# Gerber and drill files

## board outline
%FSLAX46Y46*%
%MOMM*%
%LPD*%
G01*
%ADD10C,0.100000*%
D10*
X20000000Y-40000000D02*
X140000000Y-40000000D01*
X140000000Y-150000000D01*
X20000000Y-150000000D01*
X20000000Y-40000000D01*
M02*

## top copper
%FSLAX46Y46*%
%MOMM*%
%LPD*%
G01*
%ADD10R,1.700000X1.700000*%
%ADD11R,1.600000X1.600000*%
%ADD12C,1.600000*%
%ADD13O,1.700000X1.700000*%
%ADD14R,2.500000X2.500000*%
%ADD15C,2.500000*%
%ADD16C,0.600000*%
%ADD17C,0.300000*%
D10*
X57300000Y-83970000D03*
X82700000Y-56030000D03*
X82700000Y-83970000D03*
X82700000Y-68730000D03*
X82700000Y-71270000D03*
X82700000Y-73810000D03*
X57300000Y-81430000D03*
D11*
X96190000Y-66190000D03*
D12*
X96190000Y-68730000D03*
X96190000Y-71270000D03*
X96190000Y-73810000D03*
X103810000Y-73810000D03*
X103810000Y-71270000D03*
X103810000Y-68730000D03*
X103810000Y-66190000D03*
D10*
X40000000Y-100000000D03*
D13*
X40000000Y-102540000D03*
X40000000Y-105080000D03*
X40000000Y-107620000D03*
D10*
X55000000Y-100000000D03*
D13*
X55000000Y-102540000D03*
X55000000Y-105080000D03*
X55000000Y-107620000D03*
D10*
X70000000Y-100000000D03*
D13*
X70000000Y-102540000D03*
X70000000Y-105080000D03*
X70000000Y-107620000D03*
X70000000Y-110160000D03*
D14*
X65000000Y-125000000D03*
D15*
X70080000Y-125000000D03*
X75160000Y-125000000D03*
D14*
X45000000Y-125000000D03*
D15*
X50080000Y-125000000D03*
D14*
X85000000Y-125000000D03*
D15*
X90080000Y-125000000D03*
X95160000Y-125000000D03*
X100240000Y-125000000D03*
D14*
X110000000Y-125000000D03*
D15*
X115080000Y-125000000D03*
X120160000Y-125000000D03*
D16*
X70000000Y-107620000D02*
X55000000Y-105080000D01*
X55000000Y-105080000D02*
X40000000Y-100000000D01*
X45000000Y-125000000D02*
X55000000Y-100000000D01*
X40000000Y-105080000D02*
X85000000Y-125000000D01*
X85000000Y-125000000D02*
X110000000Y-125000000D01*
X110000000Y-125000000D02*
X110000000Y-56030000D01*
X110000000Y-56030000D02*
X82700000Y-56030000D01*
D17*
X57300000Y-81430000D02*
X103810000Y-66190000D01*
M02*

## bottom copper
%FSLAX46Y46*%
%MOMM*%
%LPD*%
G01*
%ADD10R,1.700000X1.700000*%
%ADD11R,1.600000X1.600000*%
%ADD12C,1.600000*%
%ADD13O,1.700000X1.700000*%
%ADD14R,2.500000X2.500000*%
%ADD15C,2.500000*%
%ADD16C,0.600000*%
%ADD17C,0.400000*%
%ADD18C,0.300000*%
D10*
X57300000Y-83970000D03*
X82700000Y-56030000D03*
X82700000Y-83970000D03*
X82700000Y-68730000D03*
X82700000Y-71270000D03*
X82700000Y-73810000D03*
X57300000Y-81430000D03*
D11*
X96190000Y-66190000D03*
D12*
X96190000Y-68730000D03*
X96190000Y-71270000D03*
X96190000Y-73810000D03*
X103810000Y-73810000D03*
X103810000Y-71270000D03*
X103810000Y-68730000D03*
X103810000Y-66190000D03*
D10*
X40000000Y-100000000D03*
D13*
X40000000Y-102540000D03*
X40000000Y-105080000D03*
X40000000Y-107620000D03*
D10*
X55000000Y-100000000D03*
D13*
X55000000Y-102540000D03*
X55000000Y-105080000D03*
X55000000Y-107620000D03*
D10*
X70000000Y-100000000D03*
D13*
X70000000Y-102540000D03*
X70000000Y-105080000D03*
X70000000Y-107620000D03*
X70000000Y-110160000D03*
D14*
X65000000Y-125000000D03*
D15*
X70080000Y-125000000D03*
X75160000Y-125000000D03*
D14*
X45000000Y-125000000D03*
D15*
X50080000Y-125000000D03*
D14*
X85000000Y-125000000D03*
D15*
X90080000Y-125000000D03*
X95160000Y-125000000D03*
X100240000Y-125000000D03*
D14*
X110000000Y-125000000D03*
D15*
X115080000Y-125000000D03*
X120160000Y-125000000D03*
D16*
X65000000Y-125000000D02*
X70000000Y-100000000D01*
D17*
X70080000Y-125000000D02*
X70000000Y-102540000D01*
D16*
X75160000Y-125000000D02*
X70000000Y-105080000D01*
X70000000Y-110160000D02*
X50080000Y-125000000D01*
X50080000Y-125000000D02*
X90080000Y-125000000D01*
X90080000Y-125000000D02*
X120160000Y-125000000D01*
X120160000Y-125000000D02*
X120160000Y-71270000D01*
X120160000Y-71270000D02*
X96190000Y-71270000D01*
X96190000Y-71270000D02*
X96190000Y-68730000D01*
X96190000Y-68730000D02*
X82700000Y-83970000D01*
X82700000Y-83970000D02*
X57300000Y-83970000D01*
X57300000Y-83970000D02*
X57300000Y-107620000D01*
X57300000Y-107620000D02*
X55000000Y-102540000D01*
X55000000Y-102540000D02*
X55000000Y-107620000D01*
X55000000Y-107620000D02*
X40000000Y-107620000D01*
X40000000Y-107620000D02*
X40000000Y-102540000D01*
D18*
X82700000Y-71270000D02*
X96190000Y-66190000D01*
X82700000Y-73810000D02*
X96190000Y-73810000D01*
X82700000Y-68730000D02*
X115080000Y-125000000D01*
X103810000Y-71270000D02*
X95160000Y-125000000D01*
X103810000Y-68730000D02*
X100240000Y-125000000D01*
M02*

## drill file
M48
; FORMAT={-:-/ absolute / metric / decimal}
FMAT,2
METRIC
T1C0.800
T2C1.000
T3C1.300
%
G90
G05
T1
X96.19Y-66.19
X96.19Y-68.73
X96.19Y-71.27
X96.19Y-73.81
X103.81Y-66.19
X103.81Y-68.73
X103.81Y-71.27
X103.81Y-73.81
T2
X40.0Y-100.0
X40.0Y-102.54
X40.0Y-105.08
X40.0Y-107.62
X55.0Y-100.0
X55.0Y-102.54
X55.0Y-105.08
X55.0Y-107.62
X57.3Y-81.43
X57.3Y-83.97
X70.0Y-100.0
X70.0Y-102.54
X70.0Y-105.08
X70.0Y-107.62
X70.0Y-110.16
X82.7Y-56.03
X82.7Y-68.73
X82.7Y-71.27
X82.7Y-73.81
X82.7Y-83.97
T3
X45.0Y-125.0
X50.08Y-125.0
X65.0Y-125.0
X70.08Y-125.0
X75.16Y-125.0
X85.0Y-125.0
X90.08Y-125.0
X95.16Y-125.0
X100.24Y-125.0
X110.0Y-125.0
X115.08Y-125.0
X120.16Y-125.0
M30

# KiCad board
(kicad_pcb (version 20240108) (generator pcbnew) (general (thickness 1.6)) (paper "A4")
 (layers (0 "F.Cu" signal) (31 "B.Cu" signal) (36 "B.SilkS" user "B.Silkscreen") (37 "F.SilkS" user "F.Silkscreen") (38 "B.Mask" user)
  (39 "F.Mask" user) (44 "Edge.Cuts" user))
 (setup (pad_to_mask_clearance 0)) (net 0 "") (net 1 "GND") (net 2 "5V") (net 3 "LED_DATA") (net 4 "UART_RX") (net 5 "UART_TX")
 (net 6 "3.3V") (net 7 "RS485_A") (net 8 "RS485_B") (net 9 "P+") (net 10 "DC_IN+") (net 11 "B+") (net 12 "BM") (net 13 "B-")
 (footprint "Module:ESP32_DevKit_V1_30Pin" (layer "F.Cu") (at 70 70)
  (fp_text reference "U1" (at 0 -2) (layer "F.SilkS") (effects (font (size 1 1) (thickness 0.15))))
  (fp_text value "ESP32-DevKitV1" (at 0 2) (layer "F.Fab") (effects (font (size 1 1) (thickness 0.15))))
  (pad "1" thru_hole rect (at -12.7 13.97) (size 1.7 1.7) (drill 1.0) (layers "*.Cu" "*.Mask") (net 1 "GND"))
  (pad "29" thru_hole rect (at 12.7 -13.97) (size 1.7 1.7) (drill 1.0) (layers "*.Cu" "*.Mask") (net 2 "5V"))
  (pad "30" thru_hole rect (at 12.7 13.97) (size 1.7 1.7) (drill 1.0) (layers "*.Cu" "*.Mask") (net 1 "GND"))
  (pad "24" thru_hole rect (at 12.7 -1.27) (size 1.7 1.7) (drill 1.0) (layers "*.Cu" "*.Mask") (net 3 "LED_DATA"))
  (pad "25" thru_hole rect (at 12.7 1.27) (size 1.7 1.7) (drill 1.0) (layers "*.Cu" "*.Mask") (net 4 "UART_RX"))
  (pad "26" thru_hole rect (at 12.7 3.81) (size 1.7 1.7) (drill 1.0) (layers "*.Cu" "*.Mask") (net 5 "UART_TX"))
  (pad "2" thru_hole rect (at -12.7 11.43) (size 1.7 1.7) (drill 1.0) (layers "*.Cu" "*.Mask") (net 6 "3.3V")))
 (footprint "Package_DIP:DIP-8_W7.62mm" (layer "F.Cu") (at 100 70)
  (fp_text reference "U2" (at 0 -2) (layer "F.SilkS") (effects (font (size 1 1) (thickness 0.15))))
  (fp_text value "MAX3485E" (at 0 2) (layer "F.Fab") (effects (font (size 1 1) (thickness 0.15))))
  (pad "1" thru_hole rect (at -3.81 -3.81) (size 1.6 1.6) (drill 0.8) (layers "*.Cu" "*.Mask") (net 4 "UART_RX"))
  (pad "2" thru_hole circle (at -3.81 -1.27) (size 1.6 1.6) (drill 0.8) (layers "*.Cu" "*.Mask") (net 1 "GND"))
  (pad "3" thru_hole circle (at -3.81 1.27) (size 1.6 1.6) (drill 0.8) (layers "*.Cu" "*.Mask") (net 1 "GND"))
  (pad "4" thru_hole circle (at -3.81 3.81) (size 1.6 1.6) (drill 0.8) (layers "*.Cu" "*.Mask") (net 5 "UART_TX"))
  (pad "5" thru_hole circle (at 3.81 3.81) (size 1.6 1.6) (drill 0.8) (layers "*.Cu" "*.Mask") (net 1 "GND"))
  (pad "6" thru_hole circle (at 3.81 1.27) (size 1.6 1.6) (drill 0.8) (layers "*.Cu" "*.Mask") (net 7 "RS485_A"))
  (pad "7" thru_hole circle (at 3.81 -1.27) (size 1.6 1.6) (drill 0.8) (layers "*.Cu" "*.Mask") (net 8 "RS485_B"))
  (pad "8" thru_hole circle (at 3.81 -3.81) (size 1.6 1.6) (drill 0.8) (layers "*.Cu" "*.Mask") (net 6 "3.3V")))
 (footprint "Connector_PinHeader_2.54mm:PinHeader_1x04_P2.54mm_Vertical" (layer "F.Cu") (at 40 100)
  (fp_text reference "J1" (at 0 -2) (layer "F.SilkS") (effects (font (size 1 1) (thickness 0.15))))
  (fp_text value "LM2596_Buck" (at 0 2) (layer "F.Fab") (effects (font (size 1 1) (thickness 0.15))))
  (pad "1" thru_hole rect (at 0 0) (size 1.7 1.7) (drill 1.0) (layers "*.Cu" "*.Mask") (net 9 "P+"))
  (pad "2" thru_hole oval (at 0 2.54) (size 1.7 1.7) (drill 1.0) (layers "*.Cu" "*.Mask") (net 1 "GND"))
  (pad "3" thru_hole oval (at 0 5.08) (size 1.7 1.7) (drill 1.0) (layers "*.Cu" "*.Mask") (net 2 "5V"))
  (pad "4" thru_hole oval (at 0 7.62) (size 1.7 1.7) (drill 1.0) (layers "*.Cu" "*.Mask") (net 1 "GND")))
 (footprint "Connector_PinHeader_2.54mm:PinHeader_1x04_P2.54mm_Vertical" (layer "F.Cu") (at 55 100)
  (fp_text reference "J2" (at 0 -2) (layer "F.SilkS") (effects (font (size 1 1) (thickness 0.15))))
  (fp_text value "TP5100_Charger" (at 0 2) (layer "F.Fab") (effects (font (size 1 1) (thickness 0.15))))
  (pad "1" thru_hole rect (at 0 0) (size 1.7 1.7) (drill 1.0) (layers "*.Cu" "*.Mask") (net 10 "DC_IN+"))
  (pad "2" thru_hole oval (at 0 2.54) (size 1.7 1.7) (drill 1.0) (layers "*.Cu" "*.Mask") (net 1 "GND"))
  (pad "3" thru_hole oval (at 0 5.08) (size 1.7 1.7) (drill 1.0) (layers "*.Cu" "*.Mask") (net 9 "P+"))
  (pad "4" thru_hole oval (at 0 7.62) (size 1.7 1.7) (drill 1.0) (layers "*.Cu" "*.Mask") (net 1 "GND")))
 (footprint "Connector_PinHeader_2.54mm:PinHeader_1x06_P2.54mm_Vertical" (layer "F.Cu") (at 70 100)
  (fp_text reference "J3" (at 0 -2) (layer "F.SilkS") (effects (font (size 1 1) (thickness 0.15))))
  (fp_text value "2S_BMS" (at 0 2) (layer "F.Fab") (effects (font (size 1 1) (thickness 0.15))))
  (pad "1" thru_hole rect (at 0 0) (size 1.7 1.7) (drill 1.0) (layers "*.Cu" "*.Mask") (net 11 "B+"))
  (pad "2" thru_hole oval (at 0 2.54) (size 1.7 1.7) (drill 1.0) (layers "*.Cu" "*.Mask") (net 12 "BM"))
  (pad "3" thru_hole oval (at 0 5.08) (size 1.7 1.7) (drill 1.0) (layers "*.Cu" "*.Mask") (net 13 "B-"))
  (pad "4" thru_hole oval (at 0 7.62) (size 1.7 1.7) (drill 1.0) (layers "*.Cu" "*.Mask") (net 9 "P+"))
  (pad "5" thru_hole oval (at 0 10.16) (size 1.7 1.7) (drill 1.0) (layers "*.Cu" "*.Mask") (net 1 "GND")))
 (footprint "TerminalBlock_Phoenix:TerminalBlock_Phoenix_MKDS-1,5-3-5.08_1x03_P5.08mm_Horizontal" (layer "F.Cu") (at 65 125)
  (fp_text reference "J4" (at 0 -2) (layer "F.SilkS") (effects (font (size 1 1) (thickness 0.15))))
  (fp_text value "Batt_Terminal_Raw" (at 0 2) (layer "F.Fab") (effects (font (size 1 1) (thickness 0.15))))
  (pad "1" thru_hole rect (at 0 0) (size 2.5 2.5) (drill 1.3) (layers "*.Cu" "*.Mask") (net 11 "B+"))
  (pad "2" thru_hole circle (at 5.08 0) (size 2.5 2.5) (drill 1.3) (layers "*.Cu" "*.Mask") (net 12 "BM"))
  (pad "3" thru_hole circle (at 10.16 0) (size 2.5 2.5) (drill 1.3) (layers "*.Cu" "*.Mask") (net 13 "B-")))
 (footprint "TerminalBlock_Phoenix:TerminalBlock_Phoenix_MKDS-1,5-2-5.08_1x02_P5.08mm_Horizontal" (layer "F.Cu") (at 45 125)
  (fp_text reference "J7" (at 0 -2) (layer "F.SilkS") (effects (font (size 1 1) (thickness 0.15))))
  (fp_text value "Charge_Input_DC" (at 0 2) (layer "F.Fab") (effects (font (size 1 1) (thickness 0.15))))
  (pad "1" thru_hole rect (at 0 0) (size 2.5 2.5) (drill 1.3) (layers "*.Cu" "*.Mask") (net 10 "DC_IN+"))
  (pad "2" thru_hole circle (at 5.08 0) (size 2.5 2.5) (drill 1.3) (layers "*.Cu" "*.Mask") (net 1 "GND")))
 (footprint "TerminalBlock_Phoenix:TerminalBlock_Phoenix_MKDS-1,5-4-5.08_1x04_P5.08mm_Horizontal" (layer "F.Cu") (at 85 125)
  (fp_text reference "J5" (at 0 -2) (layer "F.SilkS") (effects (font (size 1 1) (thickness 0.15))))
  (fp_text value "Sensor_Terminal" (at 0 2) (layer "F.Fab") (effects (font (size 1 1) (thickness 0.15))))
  (pad "1" thru_hole rect (at 0 0) (size 2.5 2.5) (drill 1.3) (layers "*.Cu" "*.Mask") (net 2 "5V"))
  (pad "2" thru_hole circle (at 5.08 0) (size 2.5 2.5) (drill 1.3) (layers "*.Cu" "*.Mask") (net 1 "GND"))
  (pad "3" thru_hole circle (at 10.16 0) (size 2.5 2.5) (drill 1.3) (layers "*.Cu" "*.Mask") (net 7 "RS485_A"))
  (pad "4" thru_hole circle (at 15.24 0) (size 2.5 2.5) (drill 1.3) (layers "*.Cu" "*.Mask") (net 8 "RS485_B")))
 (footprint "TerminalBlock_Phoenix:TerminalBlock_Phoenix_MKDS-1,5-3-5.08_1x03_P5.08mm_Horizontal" (layer "F.Cu") (at 110 125)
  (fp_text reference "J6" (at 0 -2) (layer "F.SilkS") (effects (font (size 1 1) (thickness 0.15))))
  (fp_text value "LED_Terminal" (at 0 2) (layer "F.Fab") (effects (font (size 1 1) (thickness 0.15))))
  (pad "1" thru_hole rect (at 0 0) (size 2.5 2.5) (drill 1.3) (layers "*.Cu" "*.Mask") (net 2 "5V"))
  (pad "2" thru_hole circle (at 5.08 0) (size 2.5 2.5) (drill 1.3) (layers "*.Cu" "*.Mask") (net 3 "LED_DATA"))
  (pad "3" thru_hole circle (at 10.16 0) (size 2.5 2.5) (drill 1.3) (layers "*.Cu" "*.Mask") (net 1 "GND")))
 (segment (start 65 125) (end 70 100) (width 0.6) (layer "B.Cu") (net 11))
 (segment (start 70.08 125) (end 70 102.54) (width 0.4) (layer "B.Cu") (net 12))
 (segment (start 75.16 125) (end 70 105.08) (width 0.6) (layer "B.Cu") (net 13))
 (segment (start 70 107.62) (end 55 105.08) (width 0.6) (layer "F.Cu") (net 9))
 (segment (start 55 105.08) (end 40 100) (width 0.6) (layer "F.Cu") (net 9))
 (segment (start 45 125) (end 55 100) (width 0.6) (layer "F.Cu") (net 10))
 (segment (start 70 110.16) (end 50.08 125) (width 0.6) (layer "B.Cu") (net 1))
 (segment (start 50.08 125) (end 90.08 125) (width 0.6) (layer "B.Cu") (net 1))
 (segment (start 90.08 125) (end 120.16 125) (width 0.6) (layer "B.Cu") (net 1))
 (segment (start 120.16 125) (end 120.16 71.27) (width 0.6) (layer "B.Cu") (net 1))
 (segment (start 120.16 71.27) (end 96.19 71.27) (width 0.6) (layer "B.Cu") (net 1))
 (segment (start 96.19 71.27) (end 96.19 68.73) (width 0.6) (layer "B.Cu") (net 1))
 (segment (start 96.19 68.73) (end 82.7 83.97) (width 0.6) (layer "B.Cu") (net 1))
 (segment (start 82.7 83.97) (end 57.3 83.97) (width 0.6) (layer "B.Cu") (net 1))
 (segment (start 57.3 83.97) (end 57.3 107.62) (width 0.6) (layer "B.Cu") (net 1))
 (segment (start 57.3 107.62) (end 55 102.54) (width 0.6) (layer "B.Cu") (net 1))
 (segment (start 55 102.54) (end 55 107.62) (width 0.6) (layer "B.Cu") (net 1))
 (segment (start 55 107.62) (end 40 107.62) (width 0.6) (layer "B.Cu") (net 1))
 (segment (start 40 107.62) (end 40 102.54) (width 0.6) (layer "B.Cu") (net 1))
 (segment (start 40 105.08) (end 85 125) (width 0.6) (layer "F.Cu") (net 2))
 (segment (start 85 125) (end 110 125) (width 0.6) (layer "F.Cu") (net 2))
 (segment (start 110 125) (end 110 56.03) (width 0.6) (layer "F.Cu") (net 2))
 (segment (start 110 56.03) (end 82.7 56.03) (width 0.6) (layer "F.Cu") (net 2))
 (segment (start 57.3 81.43) (end 103.81 66.19) (width 0.3) (layer "F.Cu") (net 6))
 (segment (start 82.7 71.27) (end 96.19 66.19) (width 0.3) (layer "B.Cu") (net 4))
 (segment (start 82.7 73.81) (end 96.19 73.81) (width 0.3) (layer "B.Cu") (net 5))
 (segment (start 82.7 68.73) (end 115.08 125) (width 0.3) (layer "B.Cu") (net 3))
 (segment (start 103.81 71.27) (end 95.16 125) (width 0.3) (layer "B.Cu") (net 7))
 (segment (start 103.81 68.73) (end 100.24 125) (width 0.3) (layer "B.Cu") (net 8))
 (gr_rect (start 20 40) (end 140 150) (layer "Edge.Cuts") (width 0.1) (fill none)))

